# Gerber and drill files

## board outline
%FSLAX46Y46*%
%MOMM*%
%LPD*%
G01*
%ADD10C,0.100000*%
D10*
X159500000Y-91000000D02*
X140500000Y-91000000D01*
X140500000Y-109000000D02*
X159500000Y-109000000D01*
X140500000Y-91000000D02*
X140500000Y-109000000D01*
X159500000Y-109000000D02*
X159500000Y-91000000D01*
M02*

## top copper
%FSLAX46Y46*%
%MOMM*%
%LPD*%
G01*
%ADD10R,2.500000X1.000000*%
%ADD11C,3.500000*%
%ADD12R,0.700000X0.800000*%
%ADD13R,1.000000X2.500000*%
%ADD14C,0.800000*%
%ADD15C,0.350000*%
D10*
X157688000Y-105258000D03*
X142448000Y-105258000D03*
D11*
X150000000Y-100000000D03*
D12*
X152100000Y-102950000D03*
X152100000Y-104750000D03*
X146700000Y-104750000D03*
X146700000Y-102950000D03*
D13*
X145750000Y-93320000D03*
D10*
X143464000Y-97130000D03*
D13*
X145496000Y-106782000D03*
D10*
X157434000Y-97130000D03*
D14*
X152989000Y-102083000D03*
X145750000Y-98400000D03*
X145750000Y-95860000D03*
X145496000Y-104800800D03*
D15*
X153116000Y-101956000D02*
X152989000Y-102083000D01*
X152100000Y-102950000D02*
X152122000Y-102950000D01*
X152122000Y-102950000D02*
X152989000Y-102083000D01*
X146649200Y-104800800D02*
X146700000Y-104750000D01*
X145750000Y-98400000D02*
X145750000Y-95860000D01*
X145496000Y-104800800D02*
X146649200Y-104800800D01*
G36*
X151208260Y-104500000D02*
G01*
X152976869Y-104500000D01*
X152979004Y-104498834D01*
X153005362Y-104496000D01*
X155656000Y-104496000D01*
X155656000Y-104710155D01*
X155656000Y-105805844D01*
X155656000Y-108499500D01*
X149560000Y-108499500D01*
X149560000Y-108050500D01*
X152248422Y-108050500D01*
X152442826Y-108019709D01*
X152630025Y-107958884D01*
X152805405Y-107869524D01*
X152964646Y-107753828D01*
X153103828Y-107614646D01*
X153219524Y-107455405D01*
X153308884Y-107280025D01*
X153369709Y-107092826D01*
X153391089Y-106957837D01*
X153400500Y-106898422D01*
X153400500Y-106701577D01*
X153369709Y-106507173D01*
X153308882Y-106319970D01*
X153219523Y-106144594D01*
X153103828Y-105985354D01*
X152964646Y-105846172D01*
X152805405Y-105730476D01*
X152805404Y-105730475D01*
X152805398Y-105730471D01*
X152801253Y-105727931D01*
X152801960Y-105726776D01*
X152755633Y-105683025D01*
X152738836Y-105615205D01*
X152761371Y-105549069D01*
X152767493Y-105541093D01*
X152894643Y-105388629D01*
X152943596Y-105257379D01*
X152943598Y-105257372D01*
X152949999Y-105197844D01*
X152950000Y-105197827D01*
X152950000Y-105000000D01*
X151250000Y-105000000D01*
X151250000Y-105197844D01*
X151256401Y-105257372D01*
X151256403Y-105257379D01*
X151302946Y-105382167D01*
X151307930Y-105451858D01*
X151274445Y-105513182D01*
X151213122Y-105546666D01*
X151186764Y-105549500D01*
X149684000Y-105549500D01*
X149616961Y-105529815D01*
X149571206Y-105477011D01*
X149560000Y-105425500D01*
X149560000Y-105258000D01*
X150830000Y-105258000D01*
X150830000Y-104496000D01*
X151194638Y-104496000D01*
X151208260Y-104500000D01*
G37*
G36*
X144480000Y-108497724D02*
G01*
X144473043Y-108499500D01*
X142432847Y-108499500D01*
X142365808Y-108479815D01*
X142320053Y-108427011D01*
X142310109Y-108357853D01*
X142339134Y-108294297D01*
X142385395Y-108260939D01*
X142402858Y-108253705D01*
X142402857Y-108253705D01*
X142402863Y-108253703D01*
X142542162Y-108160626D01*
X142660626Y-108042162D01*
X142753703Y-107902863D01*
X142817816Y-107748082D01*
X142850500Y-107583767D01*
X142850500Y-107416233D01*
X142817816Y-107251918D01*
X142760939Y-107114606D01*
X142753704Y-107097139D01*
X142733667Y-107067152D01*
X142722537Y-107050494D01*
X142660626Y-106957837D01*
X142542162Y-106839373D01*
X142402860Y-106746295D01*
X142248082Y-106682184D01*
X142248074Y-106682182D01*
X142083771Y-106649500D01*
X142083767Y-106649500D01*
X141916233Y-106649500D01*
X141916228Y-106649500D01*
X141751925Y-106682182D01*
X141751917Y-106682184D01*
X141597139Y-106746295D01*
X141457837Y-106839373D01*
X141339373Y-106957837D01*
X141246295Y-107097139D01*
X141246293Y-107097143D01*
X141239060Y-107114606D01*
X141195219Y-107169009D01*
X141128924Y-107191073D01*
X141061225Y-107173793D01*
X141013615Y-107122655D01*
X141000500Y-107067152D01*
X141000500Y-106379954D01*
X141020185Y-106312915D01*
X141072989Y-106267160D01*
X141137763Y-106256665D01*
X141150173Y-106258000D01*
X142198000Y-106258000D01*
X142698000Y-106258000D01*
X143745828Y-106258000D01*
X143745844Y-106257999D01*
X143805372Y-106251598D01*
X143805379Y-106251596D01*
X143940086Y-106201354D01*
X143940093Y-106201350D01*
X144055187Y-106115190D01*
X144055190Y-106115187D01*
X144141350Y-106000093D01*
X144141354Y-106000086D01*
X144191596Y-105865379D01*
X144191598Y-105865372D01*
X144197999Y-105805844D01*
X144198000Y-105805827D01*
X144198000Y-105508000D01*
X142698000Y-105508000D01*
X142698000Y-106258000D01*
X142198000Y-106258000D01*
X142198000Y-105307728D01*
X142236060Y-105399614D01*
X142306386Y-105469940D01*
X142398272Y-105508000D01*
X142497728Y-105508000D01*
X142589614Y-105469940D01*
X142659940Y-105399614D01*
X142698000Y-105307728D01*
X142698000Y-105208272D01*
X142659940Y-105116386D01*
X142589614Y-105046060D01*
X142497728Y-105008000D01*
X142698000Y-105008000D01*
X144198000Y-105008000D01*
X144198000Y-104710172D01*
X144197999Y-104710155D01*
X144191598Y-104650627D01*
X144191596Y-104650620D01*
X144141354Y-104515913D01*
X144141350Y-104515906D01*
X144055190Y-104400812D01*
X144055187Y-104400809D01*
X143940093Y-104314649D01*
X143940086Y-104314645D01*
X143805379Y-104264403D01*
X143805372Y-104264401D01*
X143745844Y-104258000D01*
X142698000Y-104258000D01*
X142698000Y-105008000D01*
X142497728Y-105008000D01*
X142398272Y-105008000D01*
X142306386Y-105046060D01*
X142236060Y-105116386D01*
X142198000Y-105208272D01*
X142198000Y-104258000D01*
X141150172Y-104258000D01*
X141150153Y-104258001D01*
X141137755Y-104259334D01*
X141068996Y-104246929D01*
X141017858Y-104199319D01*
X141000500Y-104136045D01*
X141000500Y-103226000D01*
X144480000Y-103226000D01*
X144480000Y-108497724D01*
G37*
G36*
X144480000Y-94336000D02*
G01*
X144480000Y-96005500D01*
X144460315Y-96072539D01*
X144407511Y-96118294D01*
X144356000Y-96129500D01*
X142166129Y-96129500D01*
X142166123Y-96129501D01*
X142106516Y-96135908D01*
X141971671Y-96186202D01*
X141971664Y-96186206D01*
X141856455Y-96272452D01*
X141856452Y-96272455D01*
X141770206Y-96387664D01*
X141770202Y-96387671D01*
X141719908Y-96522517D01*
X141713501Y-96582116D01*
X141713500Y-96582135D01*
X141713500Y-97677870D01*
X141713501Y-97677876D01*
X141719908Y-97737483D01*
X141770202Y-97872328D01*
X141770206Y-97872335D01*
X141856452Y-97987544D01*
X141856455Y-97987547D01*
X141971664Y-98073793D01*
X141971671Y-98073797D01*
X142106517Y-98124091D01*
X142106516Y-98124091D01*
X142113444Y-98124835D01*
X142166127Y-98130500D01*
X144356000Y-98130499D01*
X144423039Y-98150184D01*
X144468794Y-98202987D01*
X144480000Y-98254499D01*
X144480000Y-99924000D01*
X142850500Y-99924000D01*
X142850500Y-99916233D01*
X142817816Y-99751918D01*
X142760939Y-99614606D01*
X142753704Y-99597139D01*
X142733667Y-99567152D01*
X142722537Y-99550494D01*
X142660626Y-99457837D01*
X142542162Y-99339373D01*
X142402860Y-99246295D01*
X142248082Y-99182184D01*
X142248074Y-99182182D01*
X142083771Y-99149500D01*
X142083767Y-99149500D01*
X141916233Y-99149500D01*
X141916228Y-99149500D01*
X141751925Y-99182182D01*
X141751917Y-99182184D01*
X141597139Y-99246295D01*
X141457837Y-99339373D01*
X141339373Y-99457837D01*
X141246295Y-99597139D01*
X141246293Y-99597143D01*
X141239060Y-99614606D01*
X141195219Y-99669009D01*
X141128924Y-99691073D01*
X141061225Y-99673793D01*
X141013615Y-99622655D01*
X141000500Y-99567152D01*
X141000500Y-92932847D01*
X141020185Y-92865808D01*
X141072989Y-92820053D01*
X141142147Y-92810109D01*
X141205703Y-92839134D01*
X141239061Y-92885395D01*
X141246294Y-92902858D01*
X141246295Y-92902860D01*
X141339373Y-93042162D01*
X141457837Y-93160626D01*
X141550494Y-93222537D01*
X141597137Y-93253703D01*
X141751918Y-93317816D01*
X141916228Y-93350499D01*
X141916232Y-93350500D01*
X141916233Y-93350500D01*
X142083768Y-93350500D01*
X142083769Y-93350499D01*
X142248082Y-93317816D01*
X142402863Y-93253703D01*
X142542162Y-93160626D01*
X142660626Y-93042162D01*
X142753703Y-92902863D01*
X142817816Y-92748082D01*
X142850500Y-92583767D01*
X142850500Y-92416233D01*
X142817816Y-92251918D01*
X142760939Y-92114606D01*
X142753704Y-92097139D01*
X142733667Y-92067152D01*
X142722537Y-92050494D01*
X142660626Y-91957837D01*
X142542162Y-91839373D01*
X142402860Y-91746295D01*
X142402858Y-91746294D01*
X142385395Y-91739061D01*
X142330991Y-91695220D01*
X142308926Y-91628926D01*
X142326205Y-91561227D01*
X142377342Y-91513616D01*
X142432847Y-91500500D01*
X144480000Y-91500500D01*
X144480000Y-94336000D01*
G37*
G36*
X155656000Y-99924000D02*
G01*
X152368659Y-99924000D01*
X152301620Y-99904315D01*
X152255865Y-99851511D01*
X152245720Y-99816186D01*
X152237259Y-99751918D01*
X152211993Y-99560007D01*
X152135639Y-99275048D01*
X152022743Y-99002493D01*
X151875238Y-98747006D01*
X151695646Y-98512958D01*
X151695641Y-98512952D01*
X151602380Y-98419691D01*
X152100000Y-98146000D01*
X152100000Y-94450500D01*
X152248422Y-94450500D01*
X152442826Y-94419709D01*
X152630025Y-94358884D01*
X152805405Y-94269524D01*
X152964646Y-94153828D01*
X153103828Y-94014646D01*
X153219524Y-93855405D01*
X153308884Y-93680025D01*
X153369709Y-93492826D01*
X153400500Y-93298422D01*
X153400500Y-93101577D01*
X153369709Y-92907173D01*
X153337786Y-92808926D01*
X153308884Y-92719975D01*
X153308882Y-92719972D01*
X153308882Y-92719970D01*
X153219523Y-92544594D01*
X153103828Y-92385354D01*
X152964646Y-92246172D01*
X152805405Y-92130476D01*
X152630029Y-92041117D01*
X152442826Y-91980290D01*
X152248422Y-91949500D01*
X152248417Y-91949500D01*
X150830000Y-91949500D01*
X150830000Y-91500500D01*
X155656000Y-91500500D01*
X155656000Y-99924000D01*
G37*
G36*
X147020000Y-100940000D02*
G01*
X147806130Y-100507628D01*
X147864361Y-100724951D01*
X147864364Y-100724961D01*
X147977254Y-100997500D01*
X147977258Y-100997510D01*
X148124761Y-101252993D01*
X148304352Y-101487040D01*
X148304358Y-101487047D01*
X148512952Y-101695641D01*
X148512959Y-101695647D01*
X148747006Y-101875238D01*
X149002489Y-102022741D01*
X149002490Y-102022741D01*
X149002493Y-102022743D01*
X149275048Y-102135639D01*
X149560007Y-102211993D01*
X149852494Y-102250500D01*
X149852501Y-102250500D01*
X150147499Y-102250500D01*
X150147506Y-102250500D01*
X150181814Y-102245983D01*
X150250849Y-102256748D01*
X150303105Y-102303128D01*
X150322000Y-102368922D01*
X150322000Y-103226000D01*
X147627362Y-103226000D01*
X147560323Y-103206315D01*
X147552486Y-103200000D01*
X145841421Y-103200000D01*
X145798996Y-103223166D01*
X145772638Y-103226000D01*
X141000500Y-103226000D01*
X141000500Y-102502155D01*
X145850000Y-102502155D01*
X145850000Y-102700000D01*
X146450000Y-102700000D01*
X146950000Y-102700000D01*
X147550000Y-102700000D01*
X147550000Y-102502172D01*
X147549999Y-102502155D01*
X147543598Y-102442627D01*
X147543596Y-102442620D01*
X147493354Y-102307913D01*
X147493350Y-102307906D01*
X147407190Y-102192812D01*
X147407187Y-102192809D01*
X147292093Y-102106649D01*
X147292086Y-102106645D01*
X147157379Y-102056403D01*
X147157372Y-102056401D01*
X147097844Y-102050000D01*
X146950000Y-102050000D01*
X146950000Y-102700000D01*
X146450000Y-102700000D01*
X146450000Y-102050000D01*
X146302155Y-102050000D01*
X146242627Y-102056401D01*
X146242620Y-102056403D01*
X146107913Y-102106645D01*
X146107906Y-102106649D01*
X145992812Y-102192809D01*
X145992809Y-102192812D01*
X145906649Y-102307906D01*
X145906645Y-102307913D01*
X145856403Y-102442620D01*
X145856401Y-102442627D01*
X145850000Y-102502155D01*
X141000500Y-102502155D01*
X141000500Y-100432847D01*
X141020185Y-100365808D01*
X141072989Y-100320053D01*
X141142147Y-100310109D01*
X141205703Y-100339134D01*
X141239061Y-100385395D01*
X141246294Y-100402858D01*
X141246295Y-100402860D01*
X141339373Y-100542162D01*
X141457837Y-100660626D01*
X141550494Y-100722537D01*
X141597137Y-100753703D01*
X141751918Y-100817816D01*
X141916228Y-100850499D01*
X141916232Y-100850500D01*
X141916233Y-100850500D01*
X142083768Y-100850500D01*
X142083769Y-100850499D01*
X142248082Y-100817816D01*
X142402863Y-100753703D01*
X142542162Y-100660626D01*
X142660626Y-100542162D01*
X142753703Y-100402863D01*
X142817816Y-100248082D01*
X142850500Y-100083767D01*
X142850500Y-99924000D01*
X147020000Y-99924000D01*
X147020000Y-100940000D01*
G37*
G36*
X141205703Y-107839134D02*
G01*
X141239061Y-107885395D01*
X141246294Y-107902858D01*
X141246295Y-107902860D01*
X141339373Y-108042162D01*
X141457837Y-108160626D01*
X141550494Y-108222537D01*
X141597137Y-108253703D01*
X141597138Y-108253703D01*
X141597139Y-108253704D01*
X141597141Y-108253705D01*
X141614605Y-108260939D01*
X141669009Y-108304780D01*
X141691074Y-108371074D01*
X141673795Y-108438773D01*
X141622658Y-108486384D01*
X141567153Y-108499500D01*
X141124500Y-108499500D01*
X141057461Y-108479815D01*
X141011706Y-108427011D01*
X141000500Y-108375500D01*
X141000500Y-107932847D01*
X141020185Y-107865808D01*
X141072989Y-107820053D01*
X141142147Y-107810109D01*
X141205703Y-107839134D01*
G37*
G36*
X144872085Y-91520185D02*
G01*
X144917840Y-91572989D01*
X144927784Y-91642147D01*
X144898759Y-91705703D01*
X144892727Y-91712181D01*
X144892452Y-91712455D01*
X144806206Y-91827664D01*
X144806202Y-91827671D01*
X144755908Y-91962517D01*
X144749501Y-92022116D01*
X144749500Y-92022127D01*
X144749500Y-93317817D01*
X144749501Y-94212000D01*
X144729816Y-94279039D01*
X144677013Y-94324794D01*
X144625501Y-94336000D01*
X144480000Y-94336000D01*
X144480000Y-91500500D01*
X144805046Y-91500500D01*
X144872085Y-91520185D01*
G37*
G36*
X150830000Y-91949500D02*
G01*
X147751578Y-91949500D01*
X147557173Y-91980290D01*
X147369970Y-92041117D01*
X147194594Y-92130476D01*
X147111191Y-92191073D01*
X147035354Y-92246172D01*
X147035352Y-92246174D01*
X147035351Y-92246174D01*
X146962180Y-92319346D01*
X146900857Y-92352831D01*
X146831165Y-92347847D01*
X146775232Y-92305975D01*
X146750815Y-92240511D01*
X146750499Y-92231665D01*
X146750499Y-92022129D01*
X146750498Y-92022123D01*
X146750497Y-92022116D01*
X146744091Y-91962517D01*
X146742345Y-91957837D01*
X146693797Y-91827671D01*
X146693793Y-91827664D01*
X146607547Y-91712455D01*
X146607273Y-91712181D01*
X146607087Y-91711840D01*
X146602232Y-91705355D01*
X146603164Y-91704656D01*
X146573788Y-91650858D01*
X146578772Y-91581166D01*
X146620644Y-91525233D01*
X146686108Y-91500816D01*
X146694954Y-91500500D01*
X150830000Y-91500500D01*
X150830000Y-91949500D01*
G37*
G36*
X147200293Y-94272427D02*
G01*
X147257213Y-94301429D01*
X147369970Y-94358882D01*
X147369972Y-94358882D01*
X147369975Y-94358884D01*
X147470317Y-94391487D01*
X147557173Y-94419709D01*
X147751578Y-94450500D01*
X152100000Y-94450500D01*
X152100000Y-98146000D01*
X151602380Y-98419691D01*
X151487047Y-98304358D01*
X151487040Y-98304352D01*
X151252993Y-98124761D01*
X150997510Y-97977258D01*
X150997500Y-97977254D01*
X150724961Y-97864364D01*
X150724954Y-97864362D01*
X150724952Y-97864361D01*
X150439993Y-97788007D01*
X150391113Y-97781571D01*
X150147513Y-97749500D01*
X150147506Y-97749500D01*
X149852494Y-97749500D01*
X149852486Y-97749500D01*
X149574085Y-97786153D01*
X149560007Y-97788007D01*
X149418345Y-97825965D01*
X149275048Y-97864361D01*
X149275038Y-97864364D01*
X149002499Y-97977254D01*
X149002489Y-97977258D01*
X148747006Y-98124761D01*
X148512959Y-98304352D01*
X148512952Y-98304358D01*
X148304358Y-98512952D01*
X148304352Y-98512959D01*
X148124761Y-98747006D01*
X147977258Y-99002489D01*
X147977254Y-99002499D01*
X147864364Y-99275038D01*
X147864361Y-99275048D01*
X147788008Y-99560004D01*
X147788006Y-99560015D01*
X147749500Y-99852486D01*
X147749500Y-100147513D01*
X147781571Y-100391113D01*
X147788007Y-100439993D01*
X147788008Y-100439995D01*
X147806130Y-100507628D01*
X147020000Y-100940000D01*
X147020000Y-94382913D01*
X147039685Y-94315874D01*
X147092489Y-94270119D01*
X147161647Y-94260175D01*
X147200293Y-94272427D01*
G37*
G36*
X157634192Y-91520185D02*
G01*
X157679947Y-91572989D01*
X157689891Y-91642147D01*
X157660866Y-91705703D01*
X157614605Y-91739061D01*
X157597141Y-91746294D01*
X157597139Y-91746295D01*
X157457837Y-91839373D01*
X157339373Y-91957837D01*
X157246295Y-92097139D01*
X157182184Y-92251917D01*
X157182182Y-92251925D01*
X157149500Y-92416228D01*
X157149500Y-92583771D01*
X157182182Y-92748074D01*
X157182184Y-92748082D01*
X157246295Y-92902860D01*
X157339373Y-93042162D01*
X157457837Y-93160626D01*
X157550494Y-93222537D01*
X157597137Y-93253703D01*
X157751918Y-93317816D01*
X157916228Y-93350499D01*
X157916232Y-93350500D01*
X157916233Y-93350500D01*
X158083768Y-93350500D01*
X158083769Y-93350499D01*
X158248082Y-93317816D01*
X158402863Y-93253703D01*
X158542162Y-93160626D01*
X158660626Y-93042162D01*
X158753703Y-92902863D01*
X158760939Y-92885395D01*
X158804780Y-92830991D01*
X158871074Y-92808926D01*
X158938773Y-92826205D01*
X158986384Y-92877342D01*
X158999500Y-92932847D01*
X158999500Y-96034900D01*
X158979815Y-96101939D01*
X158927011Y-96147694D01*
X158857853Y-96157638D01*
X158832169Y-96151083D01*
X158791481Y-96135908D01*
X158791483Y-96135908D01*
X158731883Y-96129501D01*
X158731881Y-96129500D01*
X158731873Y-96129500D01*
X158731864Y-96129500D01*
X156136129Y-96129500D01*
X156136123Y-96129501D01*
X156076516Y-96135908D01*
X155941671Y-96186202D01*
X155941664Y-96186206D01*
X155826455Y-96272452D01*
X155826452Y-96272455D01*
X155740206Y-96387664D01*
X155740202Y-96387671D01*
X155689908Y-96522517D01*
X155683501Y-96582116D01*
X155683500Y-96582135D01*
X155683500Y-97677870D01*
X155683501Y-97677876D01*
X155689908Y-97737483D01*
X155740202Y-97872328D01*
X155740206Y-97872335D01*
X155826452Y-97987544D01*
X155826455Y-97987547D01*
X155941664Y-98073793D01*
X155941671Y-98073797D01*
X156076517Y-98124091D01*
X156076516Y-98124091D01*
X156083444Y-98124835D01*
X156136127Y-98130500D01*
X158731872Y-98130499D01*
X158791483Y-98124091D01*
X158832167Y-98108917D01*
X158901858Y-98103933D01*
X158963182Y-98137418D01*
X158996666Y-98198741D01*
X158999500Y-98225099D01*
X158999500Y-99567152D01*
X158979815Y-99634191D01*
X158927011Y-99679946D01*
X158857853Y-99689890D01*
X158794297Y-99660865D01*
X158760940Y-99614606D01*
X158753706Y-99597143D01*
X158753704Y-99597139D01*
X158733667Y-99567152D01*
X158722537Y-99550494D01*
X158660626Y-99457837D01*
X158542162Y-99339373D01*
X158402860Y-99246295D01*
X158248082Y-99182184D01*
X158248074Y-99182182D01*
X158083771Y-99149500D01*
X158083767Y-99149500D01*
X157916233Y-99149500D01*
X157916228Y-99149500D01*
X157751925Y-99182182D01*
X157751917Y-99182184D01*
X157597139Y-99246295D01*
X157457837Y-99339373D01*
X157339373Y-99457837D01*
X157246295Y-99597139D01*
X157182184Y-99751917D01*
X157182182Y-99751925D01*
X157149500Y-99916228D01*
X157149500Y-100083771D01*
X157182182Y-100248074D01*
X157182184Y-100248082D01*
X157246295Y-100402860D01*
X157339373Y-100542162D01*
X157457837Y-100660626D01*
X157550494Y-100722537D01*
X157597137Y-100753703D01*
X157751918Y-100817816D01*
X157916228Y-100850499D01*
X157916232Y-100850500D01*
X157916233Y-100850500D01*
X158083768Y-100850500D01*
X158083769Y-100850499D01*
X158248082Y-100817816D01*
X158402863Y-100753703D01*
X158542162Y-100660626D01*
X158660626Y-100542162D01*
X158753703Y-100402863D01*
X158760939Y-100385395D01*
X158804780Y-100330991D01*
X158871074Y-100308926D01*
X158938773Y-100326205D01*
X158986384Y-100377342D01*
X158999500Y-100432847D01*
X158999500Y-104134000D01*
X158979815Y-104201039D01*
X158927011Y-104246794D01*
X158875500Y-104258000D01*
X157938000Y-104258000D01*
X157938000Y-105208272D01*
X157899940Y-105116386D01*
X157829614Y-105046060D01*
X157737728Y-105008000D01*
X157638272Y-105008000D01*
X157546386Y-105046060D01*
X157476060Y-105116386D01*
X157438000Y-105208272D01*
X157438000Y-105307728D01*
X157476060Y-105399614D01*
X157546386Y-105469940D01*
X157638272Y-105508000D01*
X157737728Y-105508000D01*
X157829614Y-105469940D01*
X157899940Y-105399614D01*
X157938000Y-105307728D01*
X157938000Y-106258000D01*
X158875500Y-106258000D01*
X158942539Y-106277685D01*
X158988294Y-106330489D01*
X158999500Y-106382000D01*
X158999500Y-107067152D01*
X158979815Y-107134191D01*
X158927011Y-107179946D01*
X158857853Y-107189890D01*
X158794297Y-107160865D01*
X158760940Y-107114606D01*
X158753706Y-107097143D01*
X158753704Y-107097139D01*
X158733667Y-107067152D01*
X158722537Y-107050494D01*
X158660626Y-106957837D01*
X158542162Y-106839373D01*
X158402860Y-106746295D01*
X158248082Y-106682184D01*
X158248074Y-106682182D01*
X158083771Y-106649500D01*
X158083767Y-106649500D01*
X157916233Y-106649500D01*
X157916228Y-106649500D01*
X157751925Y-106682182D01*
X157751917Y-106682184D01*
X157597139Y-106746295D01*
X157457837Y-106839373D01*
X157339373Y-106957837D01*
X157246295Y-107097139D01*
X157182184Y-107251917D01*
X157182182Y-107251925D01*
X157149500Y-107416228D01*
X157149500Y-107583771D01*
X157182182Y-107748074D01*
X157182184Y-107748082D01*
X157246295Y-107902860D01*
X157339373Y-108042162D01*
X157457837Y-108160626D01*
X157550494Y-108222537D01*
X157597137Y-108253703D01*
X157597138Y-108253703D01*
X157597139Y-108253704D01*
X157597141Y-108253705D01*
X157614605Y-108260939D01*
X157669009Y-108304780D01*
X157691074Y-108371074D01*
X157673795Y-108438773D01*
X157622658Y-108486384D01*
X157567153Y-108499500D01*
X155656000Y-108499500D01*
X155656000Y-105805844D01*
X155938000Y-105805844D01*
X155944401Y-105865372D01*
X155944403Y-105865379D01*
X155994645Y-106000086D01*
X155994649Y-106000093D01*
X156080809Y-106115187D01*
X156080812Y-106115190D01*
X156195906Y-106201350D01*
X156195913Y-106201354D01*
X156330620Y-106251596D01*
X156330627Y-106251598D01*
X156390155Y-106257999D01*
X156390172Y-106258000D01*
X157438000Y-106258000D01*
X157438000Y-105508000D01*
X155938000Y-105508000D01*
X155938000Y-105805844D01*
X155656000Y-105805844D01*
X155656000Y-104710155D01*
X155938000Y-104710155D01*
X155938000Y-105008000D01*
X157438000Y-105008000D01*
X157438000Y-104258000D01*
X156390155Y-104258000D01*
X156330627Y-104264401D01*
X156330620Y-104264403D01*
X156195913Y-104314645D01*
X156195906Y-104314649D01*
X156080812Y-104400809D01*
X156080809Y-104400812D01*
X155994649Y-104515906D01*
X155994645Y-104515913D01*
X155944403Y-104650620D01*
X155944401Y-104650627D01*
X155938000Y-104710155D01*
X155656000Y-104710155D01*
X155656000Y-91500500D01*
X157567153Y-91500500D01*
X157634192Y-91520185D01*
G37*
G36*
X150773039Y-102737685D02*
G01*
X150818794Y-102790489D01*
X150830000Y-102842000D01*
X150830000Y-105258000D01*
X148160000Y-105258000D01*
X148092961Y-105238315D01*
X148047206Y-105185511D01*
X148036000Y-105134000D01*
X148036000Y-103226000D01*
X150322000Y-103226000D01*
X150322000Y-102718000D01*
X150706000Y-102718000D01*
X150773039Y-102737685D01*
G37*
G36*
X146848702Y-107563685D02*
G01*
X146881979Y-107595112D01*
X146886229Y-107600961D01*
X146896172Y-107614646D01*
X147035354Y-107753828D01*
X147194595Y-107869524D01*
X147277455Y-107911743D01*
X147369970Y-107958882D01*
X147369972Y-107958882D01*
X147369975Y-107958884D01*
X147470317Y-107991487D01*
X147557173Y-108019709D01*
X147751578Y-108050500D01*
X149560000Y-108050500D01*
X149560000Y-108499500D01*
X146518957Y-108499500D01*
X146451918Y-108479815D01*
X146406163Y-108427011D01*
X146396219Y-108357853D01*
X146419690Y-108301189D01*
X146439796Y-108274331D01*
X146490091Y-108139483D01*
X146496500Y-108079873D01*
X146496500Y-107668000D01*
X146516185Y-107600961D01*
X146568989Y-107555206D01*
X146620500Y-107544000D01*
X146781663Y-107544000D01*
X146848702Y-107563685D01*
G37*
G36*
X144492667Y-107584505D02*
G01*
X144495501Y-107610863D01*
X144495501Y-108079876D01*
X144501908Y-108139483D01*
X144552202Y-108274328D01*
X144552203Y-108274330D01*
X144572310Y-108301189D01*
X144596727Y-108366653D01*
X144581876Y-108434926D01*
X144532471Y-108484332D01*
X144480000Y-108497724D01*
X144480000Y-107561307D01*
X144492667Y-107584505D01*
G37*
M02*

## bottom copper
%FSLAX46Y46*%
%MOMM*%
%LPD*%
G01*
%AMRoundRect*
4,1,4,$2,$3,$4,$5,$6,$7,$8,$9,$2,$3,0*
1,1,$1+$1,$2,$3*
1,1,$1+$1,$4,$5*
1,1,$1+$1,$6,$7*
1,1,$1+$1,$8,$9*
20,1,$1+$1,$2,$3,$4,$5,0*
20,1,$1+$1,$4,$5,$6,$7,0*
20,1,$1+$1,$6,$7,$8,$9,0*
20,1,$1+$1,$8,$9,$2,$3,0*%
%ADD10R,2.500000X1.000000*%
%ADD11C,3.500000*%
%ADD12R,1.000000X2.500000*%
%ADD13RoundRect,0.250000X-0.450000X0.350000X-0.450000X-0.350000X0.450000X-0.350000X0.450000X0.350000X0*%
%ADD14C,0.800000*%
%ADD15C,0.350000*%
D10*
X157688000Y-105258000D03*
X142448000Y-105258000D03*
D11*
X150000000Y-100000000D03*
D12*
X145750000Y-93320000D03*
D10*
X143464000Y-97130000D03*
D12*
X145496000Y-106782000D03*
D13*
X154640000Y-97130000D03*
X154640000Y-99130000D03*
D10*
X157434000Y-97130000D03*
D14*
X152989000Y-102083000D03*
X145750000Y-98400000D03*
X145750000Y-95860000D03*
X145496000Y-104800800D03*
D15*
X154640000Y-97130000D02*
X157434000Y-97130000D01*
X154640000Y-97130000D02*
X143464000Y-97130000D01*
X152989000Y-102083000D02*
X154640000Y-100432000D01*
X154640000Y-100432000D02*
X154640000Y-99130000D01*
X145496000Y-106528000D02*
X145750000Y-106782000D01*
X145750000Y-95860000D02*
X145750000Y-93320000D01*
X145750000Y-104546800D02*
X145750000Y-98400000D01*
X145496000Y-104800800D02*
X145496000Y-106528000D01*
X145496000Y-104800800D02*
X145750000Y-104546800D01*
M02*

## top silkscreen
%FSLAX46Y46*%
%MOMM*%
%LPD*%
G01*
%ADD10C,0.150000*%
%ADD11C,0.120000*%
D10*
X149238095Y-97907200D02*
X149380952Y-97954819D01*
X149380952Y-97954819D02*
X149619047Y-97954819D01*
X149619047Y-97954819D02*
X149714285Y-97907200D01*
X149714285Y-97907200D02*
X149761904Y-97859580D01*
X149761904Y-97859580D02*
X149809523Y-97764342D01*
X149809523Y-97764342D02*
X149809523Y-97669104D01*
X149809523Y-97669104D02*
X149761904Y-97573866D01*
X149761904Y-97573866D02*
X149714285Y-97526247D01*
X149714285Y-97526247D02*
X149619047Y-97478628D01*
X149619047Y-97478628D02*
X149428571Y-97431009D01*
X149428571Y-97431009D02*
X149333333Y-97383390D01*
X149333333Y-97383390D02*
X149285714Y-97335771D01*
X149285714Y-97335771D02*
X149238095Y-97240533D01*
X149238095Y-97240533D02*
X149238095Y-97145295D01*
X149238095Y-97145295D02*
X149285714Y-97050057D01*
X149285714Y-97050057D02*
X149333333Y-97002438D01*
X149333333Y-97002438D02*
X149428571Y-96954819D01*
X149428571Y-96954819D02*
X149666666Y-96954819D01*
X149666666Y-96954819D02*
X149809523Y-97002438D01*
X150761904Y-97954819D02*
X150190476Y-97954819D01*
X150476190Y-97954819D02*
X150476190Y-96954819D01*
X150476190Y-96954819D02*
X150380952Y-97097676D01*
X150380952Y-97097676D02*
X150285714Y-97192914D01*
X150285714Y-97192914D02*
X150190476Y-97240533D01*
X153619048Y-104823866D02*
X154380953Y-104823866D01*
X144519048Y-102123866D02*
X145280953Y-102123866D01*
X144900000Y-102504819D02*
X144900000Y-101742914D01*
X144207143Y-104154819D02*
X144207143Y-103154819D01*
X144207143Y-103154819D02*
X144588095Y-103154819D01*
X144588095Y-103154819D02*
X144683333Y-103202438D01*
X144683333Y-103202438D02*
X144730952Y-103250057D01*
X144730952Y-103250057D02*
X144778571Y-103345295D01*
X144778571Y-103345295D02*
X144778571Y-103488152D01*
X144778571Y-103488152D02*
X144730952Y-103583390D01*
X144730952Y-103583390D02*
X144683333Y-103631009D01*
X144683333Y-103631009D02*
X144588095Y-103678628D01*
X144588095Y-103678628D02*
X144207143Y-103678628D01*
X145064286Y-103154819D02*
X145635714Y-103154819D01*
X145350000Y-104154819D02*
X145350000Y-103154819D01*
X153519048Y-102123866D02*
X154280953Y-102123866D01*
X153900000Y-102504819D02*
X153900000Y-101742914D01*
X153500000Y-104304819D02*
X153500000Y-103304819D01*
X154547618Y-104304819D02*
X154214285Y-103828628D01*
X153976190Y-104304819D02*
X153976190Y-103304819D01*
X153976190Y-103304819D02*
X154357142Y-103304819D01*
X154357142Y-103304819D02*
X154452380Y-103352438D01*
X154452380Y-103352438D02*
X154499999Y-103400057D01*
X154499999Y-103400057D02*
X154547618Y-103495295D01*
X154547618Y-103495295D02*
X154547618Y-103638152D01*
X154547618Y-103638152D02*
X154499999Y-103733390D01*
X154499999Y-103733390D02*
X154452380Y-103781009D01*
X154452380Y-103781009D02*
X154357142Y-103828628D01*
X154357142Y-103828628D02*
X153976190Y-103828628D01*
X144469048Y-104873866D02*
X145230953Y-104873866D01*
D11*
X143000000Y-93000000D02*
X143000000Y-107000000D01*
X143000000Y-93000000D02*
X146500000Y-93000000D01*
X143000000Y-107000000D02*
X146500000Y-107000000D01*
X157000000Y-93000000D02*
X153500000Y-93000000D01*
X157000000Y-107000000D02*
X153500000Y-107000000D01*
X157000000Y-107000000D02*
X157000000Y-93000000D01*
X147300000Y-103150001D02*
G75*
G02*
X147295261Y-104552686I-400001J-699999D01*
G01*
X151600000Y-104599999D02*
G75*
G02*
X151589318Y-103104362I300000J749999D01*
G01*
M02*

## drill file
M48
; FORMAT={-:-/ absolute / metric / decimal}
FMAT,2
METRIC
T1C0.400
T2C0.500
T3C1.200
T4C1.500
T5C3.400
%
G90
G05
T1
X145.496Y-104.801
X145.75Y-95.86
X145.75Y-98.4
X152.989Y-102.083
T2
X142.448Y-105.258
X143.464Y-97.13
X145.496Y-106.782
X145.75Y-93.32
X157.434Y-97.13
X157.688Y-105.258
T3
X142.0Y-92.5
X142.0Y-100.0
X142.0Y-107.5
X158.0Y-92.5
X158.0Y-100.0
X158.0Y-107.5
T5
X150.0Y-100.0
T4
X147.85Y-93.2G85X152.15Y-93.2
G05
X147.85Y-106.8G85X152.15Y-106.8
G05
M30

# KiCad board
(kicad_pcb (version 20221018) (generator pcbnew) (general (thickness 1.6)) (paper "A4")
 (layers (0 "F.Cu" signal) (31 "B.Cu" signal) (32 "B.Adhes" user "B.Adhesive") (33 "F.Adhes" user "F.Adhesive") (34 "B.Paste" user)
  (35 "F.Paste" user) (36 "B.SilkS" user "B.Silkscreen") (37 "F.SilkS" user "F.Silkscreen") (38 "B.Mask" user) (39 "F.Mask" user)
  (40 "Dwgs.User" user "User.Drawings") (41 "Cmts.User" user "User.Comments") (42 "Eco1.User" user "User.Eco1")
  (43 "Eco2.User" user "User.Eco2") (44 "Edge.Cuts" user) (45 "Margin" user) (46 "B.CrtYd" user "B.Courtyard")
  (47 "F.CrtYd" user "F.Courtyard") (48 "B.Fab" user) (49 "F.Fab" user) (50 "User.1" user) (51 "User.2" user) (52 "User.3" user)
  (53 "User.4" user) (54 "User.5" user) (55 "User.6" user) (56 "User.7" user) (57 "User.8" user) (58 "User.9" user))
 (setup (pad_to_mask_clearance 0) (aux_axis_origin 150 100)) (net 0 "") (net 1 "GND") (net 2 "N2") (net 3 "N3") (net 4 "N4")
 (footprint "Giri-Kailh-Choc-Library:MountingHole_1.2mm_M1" (layer "F.Cu") (at 141.94 99.924)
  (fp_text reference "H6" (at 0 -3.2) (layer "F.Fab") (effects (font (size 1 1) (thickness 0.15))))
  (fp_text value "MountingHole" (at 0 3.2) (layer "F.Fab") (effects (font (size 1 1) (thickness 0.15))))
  (pad "" np_thru_hole circle (at 0.06 0.076) (size 1.2 1.2) (drill 1.2) (layers "F&B.Cu" "*.Mask")))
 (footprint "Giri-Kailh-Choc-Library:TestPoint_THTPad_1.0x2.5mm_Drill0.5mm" (layer "F.Cu") (at 157.688 105.258)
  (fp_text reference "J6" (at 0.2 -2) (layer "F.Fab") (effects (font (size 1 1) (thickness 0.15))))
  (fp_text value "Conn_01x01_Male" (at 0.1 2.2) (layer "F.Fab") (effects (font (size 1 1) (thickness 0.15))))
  (pad "1" thru_hole rect (at 0 0) (size 2.5 1) (drill 0.5) (layers "*.Cu" "*.Mask") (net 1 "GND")))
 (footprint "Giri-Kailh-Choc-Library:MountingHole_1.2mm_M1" (layer "F.Cu") (at 158.196 92.304)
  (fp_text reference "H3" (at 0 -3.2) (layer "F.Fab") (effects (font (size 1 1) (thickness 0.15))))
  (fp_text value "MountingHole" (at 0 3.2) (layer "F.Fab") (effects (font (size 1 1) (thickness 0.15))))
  (pad "" np_thru_hole circle (at -0.196 0.196) (size 1.2 1.2) (drill 1.2) (layers "F&B.Cu" "*.Mask")))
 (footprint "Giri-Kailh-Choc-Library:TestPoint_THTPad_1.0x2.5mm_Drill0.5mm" (layer "F.Cu") (at 142.448 105.258)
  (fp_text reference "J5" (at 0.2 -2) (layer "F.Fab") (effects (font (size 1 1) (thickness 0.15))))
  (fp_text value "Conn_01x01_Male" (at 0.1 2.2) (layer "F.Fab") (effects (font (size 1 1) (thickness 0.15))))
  (pad "1" thru_hole rect (at 0 0) (size 2.5 1) (drill 0.5) (layers "*.Cu" "*.Mask") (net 1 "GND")))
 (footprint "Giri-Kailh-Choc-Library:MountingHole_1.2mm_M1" (layer "F.Cu") (at 158.196 99.924)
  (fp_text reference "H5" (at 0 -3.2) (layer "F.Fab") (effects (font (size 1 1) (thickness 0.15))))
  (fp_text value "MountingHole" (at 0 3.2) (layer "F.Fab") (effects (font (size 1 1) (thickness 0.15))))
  (pad "" np_thru_hole circle (at -0.196 0.076) (size 1.2 1.2) (drill 1.2) (layers "F&B.Cu" "*.Mask")))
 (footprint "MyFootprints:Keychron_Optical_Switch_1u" (layer "F.Cu") (at 150 100)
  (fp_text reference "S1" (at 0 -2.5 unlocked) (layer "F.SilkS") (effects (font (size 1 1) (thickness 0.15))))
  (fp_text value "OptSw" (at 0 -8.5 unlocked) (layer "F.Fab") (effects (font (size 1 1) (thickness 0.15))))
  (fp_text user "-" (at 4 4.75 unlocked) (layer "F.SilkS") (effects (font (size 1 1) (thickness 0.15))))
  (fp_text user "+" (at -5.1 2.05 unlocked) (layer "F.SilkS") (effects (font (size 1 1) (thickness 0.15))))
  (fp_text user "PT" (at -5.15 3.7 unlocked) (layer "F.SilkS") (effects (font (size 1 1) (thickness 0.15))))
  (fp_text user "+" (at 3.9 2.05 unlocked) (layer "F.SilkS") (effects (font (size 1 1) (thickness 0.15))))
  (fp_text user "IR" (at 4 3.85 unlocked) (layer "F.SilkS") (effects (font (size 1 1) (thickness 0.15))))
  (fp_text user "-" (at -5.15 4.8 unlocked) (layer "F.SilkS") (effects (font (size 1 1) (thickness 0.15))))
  (fp_line (start -7 -7) (end -7 7) (stroke (width 0.12) (type solid)) (layer "F.SilkS"))
  (fp_line (start -7 -7) (end -3.5 -7) (stroke (width 0.12) (type solid)) (layer "F.SilkS"))
  (fp_line (start -7 7) (end -3.5 7) (stroke (width 0.12) (type solid)) (layer "F.SilkS"))
  (fp_line (start 7 -7) (end 3.5 -7) (stroke (width 0.12) (type solid)) (layer "F.SilkS"))
  (fp_line (start 7 7) (end 3.5 7) (stroke (width 0.12) (type solid)) (layer "F.SilkS"))
  (fp_line (start 7 7) (end 7 -7) (stroke (width 0.12) (type solid)) (layer "F.SilkS"))
  (fp_arc (start -2.7 3.150001) (mid -2.29378 3.852724) (end -2.704739 4.552686) (stroke (width 0.12) (type solid)) (layer "F.SilkS"))
  (fp_arc (start 1.6 4.599999) (mid 1.092247 3.855769) (end 1.589318 3.104362) (stroke (width 0.12) (type solid)) (layer "F.SilkS"))
  (pad "" np_thru_hole oval (at 0 -6.8) (size 5.8 1.5) (drill oval 5.8 1.5) (layers "F&B.Cu" "*.Mask") (zone_connect 2))
  (pad "" np_thru_hole circle (at 0 0) (size 3.5 3.5) (drill 3.4) (layers "F&B.Cu" "*.Mask") (zone_connect 2))
  (pad "" np_thru_hole oval (at 0 6.8) (size 5.8 1.5) (drill oval 5.8 1.5) (layers "F&B.Cu" "*.Mask") (zone_connect 2))
  (pad "1" smd rect (at 2.1 2.95) (size 0.7 0.8) (layers "F.Cu" "F.Paste" "F.Mask") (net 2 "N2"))
  (pad "2" smd rect (at 2.1 4.75) (size 0.7 0.8) (layers "F.Cu" "F.Paste" "F.Mask") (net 1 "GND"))
  (pad "3" smd rect (at -3.3 4.75) (size 0.7 0.8) (layers "F.Cu" "F.Paste" "F.Mask") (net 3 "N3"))
  (pad "4" smd rect (at -3.3 2.95) (size 0.7 0.8) (layers "F.Cu" "F.Paste" "F.Mask") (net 1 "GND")))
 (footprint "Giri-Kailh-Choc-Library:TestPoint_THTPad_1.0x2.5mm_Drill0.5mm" (layer "F.Cu") (at 145.75 93.32 90)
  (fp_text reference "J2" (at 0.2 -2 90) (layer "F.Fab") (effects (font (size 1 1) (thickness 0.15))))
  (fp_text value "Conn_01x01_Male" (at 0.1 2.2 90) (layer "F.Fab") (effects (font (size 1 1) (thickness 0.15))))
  (pad "1" thru_hole rect (at 0 0 90) (size 2.5 1) (drill 0.5) (layers "*.Cu" "*.Mask") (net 3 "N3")))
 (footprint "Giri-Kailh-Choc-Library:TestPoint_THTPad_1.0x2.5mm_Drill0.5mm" (layer "F.Cu") (at 143.464 97.13)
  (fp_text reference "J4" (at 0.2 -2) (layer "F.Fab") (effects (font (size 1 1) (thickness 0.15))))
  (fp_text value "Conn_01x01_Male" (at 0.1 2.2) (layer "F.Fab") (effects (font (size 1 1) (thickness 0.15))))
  (pad "1" thru_hole rect (at 0 0) (size 2.5 1) (drill 0.5) (layers "*.Cu" "*.Mask") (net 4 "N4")))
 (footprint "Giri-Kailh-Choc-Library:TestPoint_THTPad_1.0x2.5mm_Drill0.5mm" (layer "F.Cu") (at 145.496 106.782 90)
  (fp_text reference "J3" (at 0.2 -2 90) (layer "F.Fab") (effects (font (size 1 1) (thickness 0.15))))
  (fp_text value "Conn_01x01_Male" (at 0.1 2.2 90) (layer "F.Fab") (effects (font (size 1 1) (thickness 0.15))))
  (pad "1" thru_hole rect (at 0 0 90) (size 2.5 1) (drill 0.5) (layers "*.Cu" "*.Mask") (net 3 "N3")))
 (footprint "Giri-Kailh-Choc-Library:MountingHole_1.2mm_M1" (layer "F.Cu") (at 141.8892 92.3548)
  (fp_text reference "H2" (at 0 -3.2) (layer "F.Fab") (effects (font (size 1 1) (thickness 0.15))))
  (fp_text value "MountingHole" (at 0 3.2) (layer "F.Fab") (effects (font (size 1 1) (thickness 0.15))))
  (pad "" np_thru_hole circle (at 0.1108 0.1452) (size 1.2 1.2) (drill 1.2) (layers "F&B.Cu" "*.Mask")))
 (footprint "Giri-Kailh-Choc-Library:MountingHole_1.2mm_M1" (layer "F.Cu") (at 158.244 107.544)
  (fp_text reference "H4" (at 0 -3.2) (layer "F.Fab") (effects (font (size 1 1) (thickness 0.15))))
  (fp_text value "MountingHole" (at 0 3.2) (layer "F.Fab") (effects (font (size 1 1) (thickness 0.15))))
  (pad "" np_thru_hole circle (at -0.244 -0.044) (size 1.2 1.2) (drill 1.2) (layers "F&B.Cu" "*.Mask")))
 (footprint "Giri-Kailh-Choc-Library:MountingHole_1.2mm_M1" (layer "F.Cu") (at 141.8892 107.544)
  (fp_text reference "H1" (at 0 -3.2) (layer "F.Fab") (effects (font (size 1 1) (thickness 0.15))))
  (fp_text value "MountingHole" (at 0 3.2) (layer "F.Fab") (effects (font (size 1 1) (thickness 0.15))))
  (pad "" np_thru_hole circle (at 0.1108 -0.044) (size 1.2 1.2) (drill 1.2) (layers "F&B.Cu" "*.Mask")))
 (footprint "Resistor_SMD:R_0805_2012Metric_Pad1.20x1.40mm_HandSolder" (layer "B.Cu") (at 154.64 98.13 -90)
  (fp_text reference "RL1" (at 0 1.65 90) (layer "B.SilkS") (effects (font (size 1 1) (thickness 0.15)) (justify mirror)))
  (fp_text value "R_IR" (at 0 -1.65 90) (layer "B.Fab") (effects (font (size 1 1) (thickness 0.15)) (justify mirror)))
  (pad "1" smd roundrect (at -1 0 270) (size 1.2 1.4) (layers "B.Cu" "B.Paste" "B.Mask") (roundrect_rratio 0.2083333333) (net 4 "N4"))
  (pad "2" smd roundrect (at 1 0 270) (size 1.2 1.4) (layers "B.Cu" "B.Paste" "B.Mask") (roundrect_rratio 0.2083333333) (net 2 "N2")))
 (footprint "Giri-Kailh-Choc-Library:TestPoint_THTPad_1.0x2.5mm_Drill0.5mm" (layer "B.Cu") (at 157.434 97.13 180)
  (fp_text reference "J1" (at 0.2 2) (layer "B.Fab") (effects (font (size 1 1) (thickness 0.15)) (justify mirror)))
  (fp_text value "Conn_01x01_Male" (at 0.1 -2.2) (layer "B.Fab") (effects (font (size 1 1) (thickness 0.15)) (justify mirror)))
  (pad "1" thru_hole rect (at 0 0 180) (size 2.5 1) (drill 0.5) (layers "*.Cu" "*.Mask") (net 4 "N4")))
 (gr_line (start 159.5 91) (end 140.5 91) (stroke (width 0.1) (type default)) (layer "Edge.Cuts"))
 (gr_line (start 140.5 109) (end 159.5 109) (stroke (width 0.1) (type default)) (layer "Edge.Cuts"))
 (gr_line (start 140.5 91) (end 140.5 109) (stroke (width 0.1) (type default)) (layer "Edge.Cuts"))
 (gr_line (start 159.5 109) (end 159.5 91) (stroke (width 0.1) (type default)) (layer "Edge.Cuts"))
 (segment (start 154.64 97.13) (end 157.434 97.13) (width 0.35) (layer "B.Cu") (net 4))
 (segment (start 154.64 97.13) (end 143.464 97.13) (width 0.35) (layer "B.Cu") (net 4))
 (segment (start 153.116 101.956) (end 152.989 102.083) (width 0.35) (layer "F.Cu") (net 2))
 (segment (start 152.1 102.95) (end 152.122 102.95) (width 0.35) (layer "F.Cu") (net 2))
 (segment (start 152.122 102.95) (end 152.989 102.083) (width 0.35) (layer "F.Cu") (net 2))
 (via (at 152.989 102.083) (size 0.8) (drill 0.4) (layers "F.Cu" "B.Cu") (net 2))
 (segment (start 152.989 102.083) (end 154.64 100.432) (width 0.35) (layer "B.Cu") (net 2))
 (segment (start 154.64 100.432) (end 154.64 99.13) (width 0.35) (layer "B.Cu") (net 2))
 (segment (start 146.6492 104.8008) (end 146.7 104.75) (width 0.35) (layer "F.Cu") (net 3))
 (segment (start 145.75 98.4) (end 145.75 95.86) (width 0.35) (layer "F.Cu") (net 3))
 (segment (start 145.496 104.8008) (end 146.6492 104.8008) (width 0.35) (layer "F.Cu") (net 3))
 (via (at 145.75 98.4) (size 0.8) (drill 0.4) (layers "F.Cu" "B.Cu") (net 3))
 (via (at 145.75 95.86) (size 0.8) (drill 0.4) (layers "F.Cu" "B.Cu") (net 3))
 (via (at 145.496 104.8008) (size 0.8) (drill 0.4) (layers "F.Cu" "B.Cu") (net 3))
 (segment (start 145.496 106.528) (end 145.75 106.782) (width 0.35) (layer "B.Cu") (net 3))
 (segment (start 145.75 95.86) (end 145.75 93.32) (width 0.35) (layer "B.Cu") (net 3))
 (segment (start 145.75 104.5468) (end 145.75 98.4) (width 0.35) (layer "B.Cu") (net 3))
 (segment (start 145.496 104.8008) (end 145.496 106.528) (width 0.35) (layer "B.Cu") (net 3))
 (segment (start 145.496 104.8008) (end 145.75 104.5468) (width 0.35) (layer "B.Cu") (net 3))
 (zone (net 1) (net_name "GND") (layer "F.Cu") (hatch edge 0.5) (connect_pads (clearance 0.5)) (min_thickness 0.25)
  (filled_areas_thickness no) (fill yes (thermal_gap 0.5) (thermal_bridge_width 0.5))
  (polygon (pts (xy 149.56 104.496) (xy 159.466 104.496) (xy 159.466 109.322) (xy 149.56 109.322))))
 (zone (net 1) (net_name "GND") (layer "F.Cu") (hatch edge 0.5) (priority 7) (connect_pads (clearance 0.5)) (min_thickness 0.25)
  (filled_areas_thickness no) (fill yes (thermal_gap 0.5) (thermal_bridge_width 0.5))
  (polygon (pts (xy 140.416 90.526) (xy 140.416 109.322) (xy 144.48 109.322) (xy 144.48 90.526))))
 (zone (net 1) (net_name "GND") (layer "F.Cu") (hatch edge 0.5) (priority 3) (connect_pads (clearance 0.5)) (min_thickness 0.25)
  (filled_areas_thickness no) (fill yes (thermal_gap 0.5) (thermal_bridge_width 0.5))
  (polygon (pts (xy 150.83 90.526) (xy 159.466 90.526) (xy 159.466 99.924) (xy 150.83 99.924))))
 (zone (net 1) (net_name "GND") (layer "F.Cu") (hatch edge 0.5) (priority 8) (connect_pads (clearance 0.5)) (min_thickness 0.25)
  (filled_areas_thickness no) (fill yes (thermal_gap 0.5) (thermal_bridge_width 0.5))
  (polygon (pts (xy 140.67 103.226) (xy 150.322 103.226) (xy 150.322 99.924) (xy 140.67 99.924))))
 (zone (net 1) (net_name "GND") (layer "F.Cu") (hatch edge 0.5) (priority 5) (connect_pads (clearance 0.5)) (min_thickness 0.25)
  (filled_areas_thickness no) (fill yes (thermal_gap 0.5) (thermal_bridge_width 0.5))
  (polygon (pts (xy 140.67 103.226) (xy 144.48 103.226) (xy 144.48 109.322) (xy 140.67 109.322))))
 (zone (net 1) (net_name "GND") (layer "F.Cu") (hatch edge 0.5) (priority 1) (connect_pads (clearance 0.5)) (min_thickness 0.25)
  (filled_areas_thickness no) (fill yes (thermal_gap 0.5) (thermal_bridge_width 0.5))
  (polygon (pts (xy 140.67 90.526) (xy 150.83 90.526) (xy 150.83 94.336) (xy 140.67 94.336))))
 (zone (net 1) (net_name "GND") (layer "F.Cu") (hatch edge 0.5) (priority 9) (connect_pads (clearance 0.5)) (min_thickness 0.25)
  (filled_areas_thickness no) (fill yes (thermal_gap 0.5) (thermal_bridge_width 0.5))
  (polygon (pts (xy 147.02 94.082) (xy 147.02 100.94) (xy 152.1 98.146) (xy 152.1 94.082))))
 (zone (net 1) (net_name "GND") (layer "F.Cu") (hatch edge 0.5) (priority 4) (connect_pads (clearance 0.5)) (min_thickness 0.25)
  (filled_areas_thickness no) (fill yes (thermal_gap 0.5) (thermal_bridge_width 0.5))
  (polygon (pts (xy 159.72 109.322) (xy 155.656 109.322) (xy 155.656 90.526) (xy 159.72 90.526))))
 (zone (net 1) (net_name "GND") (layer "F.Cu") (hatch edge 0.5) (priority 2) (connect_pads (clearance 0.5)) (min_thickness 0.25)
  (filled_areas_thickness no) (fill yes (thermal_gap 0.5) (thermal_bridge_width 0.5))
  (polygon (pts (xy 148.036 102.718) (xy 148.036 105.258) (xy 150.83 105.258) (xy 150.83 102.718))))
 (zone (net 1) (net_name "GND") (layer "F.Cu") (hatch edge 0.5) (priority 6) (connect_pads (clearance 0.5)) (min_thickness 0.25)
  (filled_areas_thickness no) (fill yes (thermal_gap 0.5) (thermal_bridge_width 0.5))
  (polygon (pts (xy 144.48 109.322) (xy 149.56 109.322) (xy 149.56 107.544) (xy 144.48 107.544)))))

